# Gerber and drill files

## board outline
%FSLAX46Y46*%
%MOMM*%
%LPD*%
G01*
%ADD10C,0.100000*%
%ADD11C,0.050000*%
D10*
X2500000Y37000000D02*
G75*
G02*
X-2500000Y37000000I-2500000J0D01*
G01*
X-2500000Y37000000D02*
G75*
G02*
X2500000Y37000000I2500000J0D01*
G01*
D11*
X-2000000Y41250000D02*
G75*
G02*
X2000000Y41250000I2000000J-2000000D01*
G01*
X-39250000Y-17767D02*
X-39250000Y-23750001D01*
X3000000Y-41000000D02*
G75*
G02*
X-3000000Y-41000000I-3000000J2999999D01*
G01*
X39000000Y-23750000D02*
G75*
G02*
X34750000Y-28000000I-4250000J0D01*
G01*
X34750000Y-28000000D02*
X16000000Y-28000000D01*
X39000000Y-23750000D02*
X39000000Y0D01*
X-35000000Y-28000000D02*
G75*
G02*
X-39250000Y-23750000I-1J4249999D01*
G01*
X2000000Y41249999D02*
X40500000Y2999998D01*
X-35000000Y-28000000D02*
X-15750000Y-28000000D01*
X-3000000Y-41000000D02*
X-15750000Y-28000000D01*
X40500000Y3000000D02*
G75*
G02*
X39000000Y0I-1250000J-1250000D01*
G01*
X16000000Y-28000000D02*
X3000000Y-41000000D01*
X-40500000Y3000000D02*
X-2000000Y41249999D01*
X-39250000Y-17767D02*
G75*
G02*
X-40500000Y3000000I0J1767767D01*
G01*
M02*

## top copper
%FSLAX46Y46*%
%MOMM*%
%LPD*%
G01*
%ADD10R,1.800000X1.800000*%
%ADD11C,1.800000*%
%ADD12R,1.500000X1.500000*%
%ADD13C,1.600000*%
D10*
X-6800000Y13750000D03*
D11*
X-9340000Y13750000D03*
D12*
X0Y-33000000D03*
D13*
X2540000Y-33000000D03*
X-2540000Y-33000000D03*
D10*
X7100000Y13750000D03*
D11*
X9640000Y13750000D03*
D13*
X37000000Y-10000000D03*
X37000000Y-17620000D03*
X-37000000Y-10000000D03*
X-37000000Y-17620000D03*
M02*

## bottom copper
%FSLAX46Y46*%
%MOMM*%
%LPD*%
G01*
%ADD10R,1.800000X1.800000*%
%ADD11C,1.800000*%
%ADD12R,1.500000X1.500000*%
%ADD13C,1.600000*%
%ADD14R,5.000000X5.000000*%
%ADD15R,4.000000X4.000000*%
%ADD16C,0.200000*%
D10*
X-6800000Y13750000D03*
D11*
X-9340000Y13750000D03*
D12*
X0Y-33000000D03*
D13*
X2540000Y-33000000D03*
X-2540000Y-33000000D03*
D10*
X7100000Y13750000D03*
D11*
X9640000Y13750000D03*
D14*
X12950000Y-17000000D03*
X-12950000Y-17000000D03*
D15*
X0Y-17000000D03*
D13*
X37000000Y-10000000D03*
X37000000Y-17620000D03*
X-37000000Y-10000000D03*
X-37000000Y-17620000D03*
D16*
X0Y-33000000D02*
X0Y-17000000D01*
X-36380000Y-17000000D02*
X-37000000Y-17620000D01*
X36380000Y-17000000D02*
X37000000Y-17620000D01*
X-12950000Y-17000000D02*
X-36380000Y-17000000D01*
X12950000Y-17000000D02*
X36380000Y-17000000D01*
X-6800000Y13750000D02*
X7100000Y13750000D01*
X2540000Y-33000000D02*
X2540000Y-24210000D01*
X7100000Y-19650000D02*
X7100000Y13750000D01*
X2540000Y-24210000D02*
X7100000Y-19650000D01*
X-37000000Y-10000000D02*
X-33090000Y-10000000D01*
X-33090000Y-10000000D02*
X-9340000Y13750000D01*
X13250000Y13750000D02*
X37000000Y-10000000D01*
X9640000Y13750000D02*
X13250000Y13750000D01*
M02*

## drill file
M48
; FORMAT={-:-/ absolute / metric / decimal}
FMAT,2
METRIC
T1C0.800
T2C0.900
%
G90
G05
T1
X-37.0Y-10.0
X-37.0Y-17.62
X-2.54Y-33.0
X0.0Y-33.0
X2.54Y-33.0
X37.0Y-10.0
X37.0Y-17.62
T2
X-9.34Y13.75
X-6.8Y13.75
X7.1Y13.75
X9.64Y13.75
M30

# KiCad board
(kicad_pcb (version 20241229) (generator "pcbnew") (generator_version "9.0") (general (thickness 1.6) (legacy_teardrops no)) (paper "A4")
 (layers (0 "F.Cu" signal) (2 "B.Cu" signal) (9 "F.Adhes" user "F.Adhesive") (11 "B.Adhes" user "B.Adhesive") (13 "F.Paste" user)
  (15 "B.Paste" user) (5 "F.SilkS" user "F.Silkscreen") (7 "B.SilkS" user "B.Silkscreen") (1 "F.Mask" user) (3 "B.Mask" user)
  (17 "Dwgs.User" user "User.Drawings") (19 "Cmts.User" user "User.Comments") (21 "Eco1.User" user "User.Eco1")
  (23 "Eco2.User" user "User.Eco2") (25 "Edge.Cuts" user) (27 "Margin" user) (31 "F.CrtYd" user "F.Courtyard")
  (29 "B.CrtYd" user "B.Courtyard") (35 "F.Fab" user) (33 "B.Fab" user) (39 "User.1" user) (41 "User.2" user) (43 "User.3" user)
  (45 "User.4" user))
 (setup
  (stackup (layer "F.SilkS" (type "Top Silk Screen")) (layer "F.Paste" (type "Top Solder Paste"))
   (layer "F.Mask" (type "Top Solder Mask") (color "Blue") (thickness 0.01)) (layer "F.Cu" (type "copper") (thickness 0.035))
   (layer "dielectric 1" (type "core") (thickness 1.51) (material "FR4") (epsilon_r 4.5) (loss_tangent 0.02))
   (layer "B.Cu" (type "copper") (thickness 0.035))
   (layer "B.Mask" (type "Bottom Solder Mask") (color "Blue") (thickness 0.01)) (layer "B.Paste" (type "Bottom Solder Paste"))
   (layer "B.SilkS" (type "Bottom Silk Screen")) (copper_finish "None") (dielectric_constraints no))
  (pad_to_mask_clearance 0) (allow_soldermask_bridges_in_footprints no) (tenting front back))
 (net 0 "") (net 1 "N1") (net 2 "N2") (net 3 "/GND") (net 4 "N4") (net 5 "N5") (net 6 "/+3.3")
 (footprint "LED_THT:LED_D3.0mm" (layer "F.Cu") (at -6.8 -13.75 180)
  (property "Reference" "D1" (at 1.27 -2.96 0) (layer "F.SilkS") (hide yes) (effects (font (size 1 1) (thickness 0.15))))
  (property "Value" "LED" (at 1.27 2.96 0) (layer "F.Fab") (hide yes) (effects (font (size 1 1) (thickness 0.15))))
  (pad "1" thru_hole rect (at 0 0 180) (size 1.8 1.8) (drill 0.9) (layers "*.Cu" "*.Mask") (remove_unused_layers no) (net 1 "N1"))
  (pad "2" thru_hole circle (at 2.54 0 180) (size 1.8 1.8) (drill 0.9) (layers "*.Cu" "*.Mask") (remove_unused_layers no) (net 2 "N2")))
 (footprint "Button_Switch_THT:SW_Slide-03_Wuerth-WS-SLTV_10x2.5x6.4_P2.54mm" (layer "F.Cu") (at 0 33 180)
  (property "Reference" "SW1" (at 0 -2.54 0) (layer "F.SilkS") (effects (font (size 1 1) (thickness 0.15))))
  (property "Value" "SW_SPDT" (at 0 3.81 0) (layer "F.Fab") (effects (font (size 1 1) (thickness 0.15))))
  (pad "1" thru_hole rect (at 0 0 180) (size 1.5 1.5) (drill 0.8) (layers "*.Cu" "*.Mask") (remove_unused_layers no) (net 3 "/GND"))
  (pad "2" thru_hole circle (at -2.54 0 180) (size 1.6 1.6) (drill 0.8) (layers "*.Cu" "*.Mask") (remove_unused_layers no) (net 1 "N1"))
  (pad "3" thru_hole circle (at 2.54 0 180) (size 1.6 1.6) (drill 0.8) (layers "*.Cu" "*.Mask") (remove_unused_layers no) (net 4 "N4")))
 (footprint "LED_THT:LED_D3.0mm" (layer "F.Cu") (at 7.1 -13.75)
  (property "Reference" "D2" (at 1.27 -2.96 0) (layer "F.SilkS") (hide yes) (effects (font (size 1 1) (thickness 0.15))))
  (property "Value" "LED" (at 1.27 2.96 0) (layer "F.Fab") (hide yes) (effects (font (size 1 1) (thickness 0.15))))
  (pad "1" thru_hole rect (at 0 0) (size 1.8 1.8) (drill 0.9) (layers "*.Cu" "*.Mask") (remove_unused_layers no) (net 1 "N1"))
  (pad "2" thru_hole circle (at 2.54 0) (size 1.8 1.8) (drill 0.9) (layers "*.Cu" "*.Mask") (remove_unused_layers no) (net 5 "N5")))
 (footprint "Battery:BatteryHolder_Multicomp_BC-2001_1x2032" (layer "B.Cu") (at 0 17 180)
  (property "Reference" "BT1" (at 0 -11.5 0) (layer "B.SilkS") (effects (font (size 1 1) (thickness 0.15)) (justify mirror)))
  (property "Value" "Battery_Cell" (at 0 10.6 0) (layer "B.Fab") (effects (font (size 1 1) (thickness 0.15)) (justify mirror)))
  (pad "1" smd rect (at -12.95 0 180) (size 5 5) (layers "B.Cu" "B.Mask" "B.Paste") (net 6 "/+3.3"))
  (pad "1" smd rect (at 12.95 0 180) (size 5 5) (layers "B.Cu" "B.Mask" "B.Paste") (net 6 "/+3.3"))
  (pad "2" smd rect (at 0 0 180) (size 4 4) (layers "B.Cu" "B.Mask" "B.Paste") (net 3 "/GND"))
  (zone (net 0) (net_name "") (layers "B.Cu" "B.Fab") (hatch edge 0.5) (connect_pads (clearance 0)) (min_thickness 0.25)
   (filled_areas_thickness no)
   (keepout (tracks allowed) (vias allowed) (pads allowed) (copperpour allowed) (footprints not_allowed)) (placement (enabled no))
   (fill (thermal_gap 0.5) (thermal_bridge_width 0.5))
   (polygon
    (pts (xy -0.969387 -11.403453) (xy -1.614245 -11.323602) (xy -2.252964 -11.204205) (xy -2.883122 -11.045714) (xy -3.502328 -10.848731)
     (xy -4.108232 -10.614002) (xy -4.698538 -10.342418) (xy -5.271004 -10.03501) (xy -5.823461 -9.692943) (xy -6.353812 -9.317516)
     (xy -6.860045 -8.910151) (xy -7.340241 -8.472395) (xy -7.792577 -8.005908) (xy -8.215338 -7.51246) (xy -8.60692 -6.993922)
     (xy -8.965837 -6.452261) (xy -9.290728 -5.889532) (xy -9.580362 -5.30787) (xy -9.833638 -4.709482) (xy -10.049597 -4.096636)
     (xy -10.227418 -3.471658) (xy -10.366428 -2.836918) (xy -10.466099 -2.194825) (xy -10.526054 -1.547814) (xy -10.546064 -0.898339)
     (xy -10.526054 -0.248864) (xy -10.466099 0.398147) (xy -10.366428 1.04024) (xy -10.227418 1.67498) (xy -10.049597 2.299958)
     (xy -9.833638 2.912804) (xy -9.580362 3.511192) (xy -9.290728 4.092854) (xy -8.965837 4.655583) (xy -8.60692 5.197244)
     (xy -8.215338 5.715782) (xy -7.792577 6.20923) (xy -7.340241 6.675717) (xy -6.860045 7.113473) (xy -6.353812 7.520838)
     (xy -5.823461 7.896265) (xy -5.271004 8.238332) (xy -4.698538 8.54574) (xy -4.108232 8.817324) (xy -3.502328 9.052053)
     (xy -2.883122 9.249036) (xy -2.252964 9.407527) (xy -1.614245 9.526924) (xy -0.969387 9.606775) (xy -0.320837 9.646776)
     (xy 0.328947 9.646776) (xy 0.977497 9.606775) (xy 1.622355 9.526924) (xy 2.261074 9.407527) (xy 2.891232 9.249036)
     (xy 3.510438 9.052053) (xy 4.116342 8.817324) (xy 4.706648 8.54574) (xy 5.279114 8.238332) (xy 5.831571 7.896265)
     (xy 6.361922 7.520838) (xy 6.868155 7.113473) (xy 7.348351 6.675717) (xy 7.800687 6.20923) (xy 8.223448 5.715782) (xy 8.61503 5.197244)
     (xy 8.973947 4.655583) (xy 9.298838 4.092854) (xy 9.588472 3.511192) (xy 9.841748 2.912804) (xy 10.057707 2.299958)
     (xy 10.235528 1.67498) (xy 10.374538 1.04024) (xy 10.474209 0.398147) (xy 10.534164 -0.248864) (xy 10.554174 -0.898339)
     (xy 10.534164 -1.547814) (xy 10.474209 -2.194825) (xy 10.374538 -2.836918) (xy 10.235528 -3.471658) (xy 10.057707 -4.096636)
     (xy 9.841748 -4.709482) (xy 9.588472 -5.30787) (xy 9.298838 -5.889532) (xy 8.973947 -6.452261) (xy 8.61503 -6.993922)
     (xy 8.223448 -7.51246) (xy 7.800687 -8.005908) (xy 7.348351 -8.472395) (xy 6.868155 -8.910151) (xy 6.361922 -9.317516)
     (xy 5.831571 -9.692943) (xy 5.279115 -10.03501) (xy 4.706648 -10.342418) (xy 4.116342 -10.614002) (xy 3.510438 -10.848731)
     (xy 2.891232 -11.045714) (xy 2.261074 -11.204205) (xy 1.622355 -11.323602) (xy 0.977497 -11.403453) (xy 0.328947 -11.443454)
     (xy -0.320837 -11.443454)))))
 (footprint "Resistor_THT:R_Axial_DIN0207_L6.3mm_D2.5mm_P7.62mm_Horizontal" (layer "B.Cu") (at 37 10 -90)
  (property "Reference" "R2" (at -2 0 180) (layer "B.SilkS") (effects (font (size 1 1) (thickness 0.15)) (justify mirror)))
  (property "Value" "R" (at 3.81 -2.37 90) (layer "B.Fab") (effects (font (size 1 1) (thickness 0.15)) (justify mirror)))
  (pad "1" thru_hole circle (at 0 0 270) (size 1.6 1.6) (drill 0.8) (layers "*.Cu" "*.Mask") (remove_unused_layers no) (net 5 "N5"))
  (pad "2" thru_hole circle (at 7.62 0 270) (size 1.6 1.6) (drill 0.8) (layers "*.Cu" "*.Mask") (remove_unused_layers no) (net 6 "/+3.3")))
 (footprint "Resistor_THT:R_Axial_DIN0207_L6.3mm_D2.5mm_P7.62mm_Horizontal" (layer "B.Cu") (at -37 10 -90)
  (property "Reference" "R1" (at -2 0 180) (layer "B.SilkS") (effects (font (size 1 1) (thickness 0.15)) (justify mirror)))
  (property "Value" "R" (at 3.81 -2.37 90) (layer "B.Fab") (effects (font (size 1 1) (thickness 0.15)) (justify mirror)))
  (pad "1" thru_hole circle (at 0 0 270) (size 1.6 1.6) (drill 0.8) (layers "*.Cu" "*.Mask") (remove_unused_layers no) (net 2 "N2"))
  (pad "2" thru_hole circle (at 7.62 0 270) (size 1.6 1.6) (drill 0.8) (layers "*.Cu" "*.Mask") (remove_unused_layers no) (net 6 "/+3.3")))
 (gr_circle (center 0 -37) (end 2.5 -37) (stroke (width 0.1) (type solid)) (fill no) (layer "Edge.Cuts"))
 (gr_arc (start -2 -41.25) (mid 0 -42.078427) (end 2 -41.25) (stroke (width 0.05) (type default)) (layer "Edge.Cuts"))
 (gr_line (start -39.25 0.017767) (end -39.25 23.750001) (stroke (width 0.05) (type default)) (layer "Edge.Cuts"))
 (gr_arc (start 3 41) (mid 0 42.242641) (end -3 41) (stroke (width 0.05) (type default)) (layer "Edge.Cuts"))
 (gr_arc (start 39 23.75) (mid 37.755204 26.755204) (end 34.75 28) (stroke (width 0.05) (type default)) (layer "Edge.Cuts"))
 (gr_line (start 34.75 28) (end 16 28) (stroke (width 0.05) (type default)) (layer "Edge.Cuts"))
 (gr_line (start 39 23.75) (end 39 0) (stroke (width 0.05) (type default)) (layer "Edge.Cuts"))
 (gr_arc (start -35 28) (mid -38.005204 26.755204) (end -39.25 23.75) (stroke (width 0.05) (type default)) (layer "Edge.Cuts"))
 (gr_line (start 2 -41.249999) (end 40.5 -2.999998) (stroke (width 0.05) (type default)) (layer "Edge.Cuts"))
 (gr_line (start -35 28) (end -15.75 28) (stroke (width 0.05) (type default)) (layer "Edge.Cuts"))
 (gr_line (start -3 41) (end -15.75 28) (stroke (width 0.05) (type default)) (layer "Edge.Cuts"))
 (gr_arc (start 40.5 -3) (mid 40.831139 -0.959431) (end 39 0) (stroke (width 0.05) (type default)) (layer "Edge.Cuts"))
 (gr_line (start 16 28) (end 3 41) (stroke (width 0.05) (type default)) (layer "Edge.Cuts"))
 (gr_line (start -40.5 -3) (end -2 -41.249999) (stroke (width 0.05) (type default)) (layer "Edge.Cuts"))
 (gr_arc (start -39.25 0.017767) (mid -40.883204 -1.073505) (end -40.5 -3) (stroke (width 0.05) (type default)) (layer "Edge.Cuts"))
 (segment (start 0 33) (end 0 17) (width 0.2) (layer "B.Cu") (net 3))
 (segment (start -36.38 17) (end -37 17.62) (width 0.2) (layer "B.Cu") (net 6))
 (segment (start 36.38 17) (end 37 17.62) (width 0.2) (layer "B.Cu") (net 6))
 (segment (start -12.95 17) (end -36.38 17) (width 0.2) (layer "B.Cu") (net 6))
 (segment (start 12.95 17) (end 36.38 17) (width 0.2) (layer "B.Cu") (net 6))
 (segment (start -6.8 -13.75) (end 7.1 -13.75) (width 0.2) (layer "B.Cu") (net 1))
 (segment (start 2.54 33) (end 2.54 24.21) (width 0.2) (layer "B.Cu") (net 1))
 (segment (start 7.1 19.65) (end 7.1 -13.75) (width 0.2) (layer "B.Cu") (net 1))
 (segment (start 2.54 24.21) (end 7.1 19.65) (width 0.2) (layer "B.Cu") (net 1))
 (segment (start -37 10) (end -33.09 10) (width 0.2) (layer "B.Cu") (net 2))
 (segment (start -33.09 10) (end -9.34 -13.75) (width 0.2) (layer "B.Cu") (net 2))
 (segment (start 13.25 -13.75) (end 37 10) (width 0.2) (layer "B.Cu") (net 5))
 (segment (start 9.64 -13.75) (end 13.25 -13.75) (width 0.2) (layer "B.Cu") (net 5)))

